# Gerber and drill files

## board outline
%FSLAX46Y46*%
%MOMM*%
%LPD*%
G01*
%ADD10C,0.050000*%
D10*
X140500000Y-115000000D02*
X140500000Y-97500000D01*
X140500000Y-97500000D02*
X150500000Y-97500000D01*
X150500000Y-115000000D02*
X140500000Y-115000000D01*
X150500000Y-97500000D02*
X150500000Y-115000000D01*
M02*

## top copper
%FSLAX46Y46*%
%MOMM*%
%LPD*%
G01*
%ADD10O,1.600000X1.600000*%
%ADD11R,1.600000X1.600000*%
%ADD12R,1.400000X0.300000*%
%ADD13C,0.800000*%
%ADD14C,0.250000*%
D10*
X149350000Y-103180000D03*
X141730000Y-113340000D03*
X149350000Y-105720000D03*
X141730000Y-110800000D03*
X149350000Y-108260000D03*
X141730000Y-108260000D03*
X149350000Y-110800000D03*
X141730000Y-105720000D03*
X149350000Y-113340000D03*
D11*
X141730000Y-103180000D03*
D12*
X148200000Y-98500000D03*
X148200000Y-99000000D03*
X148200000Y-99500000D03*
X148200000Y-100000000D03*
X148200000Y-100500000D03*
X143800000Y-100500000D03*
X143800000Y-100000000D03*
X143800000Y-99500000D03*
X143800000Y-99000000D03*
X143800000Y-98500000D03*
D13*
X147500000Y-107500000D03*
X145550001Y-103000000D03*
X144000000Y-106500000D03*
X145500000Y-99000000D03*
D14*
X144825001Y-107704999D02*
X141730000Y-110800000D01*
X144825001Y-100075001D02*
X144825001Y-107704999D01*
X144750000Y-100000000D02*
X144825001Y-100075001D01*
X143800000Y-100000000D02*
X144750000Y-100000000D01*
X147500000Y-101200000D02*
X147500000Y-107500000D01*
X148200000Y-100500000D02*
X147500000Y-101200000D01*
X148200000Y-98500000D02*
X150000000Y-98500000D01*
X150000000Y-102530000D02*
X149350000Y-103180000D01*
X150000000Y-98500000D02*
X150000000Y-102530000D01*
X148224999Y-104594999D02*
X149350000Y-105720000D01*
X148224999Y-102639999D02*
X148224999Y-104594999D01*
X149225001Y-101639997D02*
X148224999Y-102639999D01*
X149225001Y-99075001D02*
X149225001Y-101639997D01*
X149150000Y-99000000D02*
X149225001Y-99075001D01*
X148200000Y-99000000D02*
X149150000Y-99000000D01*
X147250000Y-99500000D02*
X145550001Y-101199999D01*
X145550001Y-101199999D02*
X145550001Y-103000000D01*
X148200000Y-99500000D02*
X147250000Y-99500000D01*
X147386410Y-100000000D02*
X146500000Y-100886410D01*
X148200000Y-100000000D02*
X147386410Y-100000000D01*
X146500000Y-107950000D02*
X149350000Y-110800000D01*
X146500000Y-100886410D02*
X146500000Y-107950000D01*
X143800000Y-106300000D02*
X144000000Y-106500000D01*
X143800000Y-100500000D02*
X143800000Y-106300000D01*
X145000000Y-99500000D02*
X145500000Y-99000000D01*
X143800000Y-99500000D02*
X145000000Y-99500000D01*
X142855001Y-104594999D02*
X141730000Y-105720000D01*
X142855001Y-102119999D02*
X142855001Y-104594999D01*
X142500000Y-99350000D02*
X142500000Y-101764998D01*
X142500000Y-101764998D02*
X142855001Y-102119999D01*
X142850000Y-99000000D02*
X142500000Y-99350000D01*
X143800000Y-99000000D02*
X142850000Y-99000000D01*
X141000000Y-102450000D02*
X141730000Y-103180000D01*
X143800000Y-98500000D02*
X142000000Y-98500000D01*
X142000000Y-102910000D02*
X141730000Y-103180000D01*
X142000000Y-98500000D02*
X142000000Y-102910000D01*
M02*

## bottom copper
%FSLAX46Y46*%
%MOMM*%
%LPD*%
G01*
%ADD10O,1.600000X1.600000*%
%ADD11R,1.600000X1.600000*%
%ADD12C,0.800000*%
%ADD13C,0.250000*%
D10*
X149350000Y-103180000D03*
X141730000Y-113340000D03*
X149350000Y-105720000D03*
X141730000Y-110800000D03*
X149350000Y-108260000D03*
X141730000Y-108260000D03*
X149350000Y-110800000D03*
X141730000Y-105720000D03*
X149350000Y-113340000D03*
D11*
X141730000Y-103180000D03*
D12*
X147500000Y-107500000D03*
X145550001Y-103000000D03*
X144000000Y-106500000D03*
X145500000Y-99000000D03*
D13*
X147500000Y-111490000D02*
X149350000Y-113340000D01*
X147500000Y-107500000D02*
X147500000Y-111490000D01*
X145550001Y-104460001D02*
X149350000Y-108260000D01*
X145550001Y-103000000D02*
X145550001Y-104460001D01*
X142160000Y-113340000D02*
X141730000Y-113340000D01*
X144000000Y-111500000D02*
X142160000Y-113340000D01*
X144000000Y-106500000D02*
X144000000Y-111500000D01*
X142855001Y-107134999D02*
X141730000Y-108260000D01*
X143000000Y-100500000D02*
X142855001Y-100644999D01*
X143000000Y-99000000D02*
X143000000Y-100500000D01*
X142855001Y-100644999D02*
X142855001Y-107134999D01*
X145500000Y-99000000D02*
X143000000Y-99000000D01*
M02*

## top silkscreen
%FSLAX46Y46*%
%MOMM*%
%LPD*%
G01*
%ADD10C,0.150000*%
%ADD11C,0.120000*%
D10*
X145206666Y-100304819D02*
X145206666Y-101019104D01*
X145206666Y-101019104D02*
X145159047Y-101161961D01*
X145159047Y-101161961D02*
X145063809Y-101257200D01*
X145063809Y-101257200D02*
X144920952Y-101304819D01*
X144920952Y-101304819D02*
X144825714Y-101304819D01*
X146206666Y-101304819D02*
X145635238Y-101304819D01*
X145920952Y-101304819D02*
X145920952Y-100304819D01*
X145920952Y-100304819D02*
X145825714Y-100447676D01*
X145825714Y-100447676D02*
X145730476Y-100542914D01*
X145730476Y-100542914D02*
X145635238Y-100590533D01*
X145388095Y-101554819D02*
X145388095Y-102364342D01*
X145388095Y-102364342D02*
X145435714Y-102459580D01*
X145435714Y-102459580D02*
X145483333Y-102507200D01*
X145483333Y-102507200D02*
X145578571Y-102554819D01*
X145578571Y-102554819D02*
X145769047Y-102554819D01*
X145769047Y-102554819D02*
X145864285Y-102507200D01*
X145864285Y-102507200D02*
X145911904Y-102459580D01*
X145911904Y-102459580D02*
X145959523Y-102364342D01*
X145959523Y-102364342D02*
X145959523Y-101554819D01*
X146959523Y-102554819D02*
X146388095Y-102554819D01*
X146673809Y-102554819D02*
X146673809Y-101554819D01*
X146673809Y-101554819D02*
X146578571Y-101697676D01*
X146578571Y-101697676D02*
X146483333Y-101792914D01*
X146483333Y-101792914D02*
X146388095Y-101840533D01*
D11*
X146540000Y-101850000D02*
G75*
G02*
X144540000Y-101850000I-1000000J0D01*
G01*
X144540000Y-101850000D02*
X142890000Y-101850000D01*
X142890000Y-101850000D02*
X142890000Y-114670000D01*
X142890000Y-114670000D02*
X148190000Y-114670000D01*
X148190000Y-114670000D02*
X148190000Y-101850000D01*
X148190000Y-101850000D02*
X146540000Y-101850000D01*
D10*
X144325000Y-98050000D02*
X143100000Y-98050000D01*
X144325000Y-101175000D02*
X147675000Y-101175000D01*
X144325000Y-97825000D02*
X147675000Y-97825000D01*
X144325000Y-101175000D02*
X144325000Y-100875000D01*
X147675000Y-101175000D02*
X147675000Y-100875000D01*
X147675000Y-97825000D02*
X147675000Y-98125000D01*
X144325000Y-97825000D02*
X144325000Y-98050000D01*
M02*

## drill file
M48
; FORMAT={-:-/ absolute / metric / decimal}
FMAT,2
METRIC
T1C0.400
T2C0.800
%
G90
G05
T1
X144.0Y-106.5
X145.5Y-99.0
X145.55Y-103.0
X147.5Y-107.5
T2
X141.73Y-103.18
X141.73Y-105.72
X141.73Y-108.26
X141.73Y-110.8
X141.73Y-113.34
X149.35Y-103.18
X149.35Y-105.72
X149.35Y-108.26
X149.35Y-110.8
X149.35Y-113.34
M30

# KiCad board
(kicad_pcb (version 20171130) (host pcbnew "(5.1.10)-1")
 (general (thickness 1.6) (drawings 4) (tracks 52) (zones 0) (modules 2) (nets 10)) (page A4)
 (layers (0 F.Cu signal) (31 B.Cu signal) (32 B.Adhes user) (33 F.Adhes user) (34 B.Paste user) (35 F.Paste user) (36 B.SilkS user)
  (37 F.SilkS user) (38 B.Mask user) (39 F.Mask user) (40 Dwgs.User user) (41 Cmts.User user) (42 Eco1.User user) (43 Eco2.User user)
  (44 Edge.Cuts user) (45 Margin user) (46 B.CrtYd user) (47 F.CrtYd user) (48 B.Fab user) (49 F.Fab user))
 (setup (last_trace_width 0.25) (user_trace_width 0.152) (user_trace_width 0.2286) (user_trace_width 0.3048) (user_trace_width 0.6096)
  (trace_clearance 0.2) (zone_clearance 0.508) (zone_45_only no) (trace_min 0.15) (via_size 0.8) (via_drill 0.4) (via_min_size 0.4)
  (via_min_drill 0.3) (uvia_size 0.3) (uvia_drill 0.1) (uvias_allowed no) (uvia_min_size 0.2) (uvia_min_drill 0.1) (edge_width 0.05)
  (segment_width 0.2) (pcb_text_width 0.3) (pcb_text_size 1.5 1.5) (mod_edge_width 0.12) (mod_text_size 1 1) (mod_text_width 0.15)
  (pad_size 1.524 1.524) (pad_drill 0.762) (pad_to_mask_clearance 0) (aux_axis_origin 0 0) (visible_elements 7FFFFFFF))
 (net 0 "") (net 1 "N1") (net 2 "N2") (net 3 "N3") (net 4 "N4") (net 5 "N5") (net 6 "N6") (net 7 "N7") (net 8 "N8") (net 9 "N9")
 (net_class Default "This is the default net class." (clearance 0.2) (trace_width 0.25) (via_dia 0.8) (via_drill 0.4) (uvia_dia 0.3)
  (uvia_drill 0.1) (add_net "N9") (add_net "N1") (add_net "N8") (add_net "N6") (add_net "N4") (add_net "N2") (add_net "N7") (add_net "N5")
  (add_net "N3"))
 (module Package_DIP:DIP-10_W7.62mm (layer F.Cu) (at 141.73 103.18)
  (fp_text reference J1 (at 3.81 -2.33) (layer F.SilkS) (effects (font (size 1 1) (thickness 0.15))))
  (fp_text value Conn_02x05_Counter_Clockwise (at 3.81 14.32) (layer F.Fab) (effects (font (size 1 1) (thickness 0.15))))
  (fp_arc (start 3.81 -1.33) (end 2.81 -1.33) (angle -180) (layer F.SilkS) (width 0.12))
  (fp_line (start 2.81 -1.33) (end 1.16 -1.33) (layer F.SilkS) (width 0.12))
  (fp_line (start 1.16 -1.33) (end 1.16 11.49) (layer F.SilkS) (width 0.12))
  (fp_line (start 1.16 11.49) (end 6.46 11.49) (layer F.SilkS) (width 0.12))
  (fp_line (start 6.46 11.49) (end 6.46 -1.33) (layer F.SilkS) (width 0.12))
  (fp_line (start 6.46 -1.33) (end 4.81 -1.33) (layer F.SilkS) (width 0.12))
  (pad 10 thru_hole oval (at 7.62 0) (size 1.6 1.6) (drill 0.8) (layers *.Cu *.Mask) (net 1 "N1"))
  (pad 5 thru_hole oval (at 0 10.16) (size 1.6 1.6) (drill 0.8) (layers *.Cu *.Mask) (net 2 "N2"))
  (pad 9 thru_hole oval (at 7.62 2.54) (size 1.6 1.6) (drill 0.8) (layers *.Cu *.Mask) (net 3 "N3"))
  (pad 4 thru_hole oval (at 0 7.62) (size 1.6 1.6) (drill 0.8) (layers *.Cu *.Mask) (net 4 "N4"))
  (pad 8 thru_hole oval (at 7.62 5.08) (size 1.6 1.6) (drill 0.8) (layers *.Cu *.Mask) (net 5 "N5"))
  (pad 3 thru_hole oval (at 0 5.08) (size 1.6 1.6) (drill 0.8) (layers *.Cu *.Mask) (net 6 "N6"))
  (pad 7 thru_hole oval (at 7.62 7.62) (size 1.6 1.6) (drill 0.8) (layers *.Cu *.Mask) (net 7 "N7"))
  (pad 2 thru_hole oval (at 0 2.54) (size 1.6 1.6) (drill 0.8) (layers *.Cu *.Mask) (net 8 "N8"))
  (pad 6 thru_hole oval (at 7.62 10.16) (size 1.6 1.6) (drill 0.8) (layers *.Cu *.Mask) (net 4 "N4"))
  (pad 1 thru_hole rect (at 0 0) (size 1.6 1.6) (drill 0.8) (layers *.Cu *.Mask) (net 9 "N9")))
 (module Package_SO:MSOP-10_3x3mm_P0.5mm (layer F.Cu) (at 146 99.5)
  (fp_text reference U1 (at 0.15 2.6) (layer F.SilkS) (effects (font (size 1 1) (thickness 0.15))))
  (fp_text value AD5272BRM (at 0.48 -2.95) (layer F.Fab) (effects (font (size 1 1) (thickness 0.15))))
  (fp_line (start -1.675 -1.45) (end -2.9 -1.45) (layer F.SilkS) (width 0.15))
  (fp_line (start -1.675 1.675) (end 1.675 1.675) (layer F.SilkS) (width 0.15))
  (fp_line (start -1.675 -1.675) (end 1.675 -1.675) (layer F.SilkS) (width 0.15))
  (fp_line (start -1.675 1.675) (end -1.675 1.375) (layer F.SilkS) (width 0.15))
  (fp_line (start 1.675 1.675) (end 1.675 1.375) (layer F.SilkS) (width 0.15))
  (fp_line (start 1.675 -1.675) (end 1.675 -1.375) (layer F.SilkS) (width 0.15))
  (fp_line (start -1.675 -1.675) (end -1.675 -1.45) (layer F.SilkS) (width 0.15))
  (pad 10 smd rect (at 2.2 -1) (size 1.4 0.3) (layers F.Cu F.Paste F.Mask) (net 1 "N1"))
  (pad 9 smd rect (at 2.2 -0.5) (size 1.4 0.3) (layers F.Cu F.Paste F.Mask) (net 3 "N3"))
  (pad 8 smd rect (at 2.2 0) (size 1.4 0.3) (layers F.Cu F.Paste F.Mask) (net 5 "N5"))
  (pad 7 smd rect (at 2.2 0.5) (size 1.4 0.3) (layers F.Cu F.Paste F.Mask) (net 7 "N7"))
  (pad 6 smd rect (at 2.2 1) (size 1.4 0.3) (layers F.Cu F.Paste F.Mask) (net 4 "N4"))
  (pad 5 smd rect (at -2.2 1) (size 1.4 0.3) (layers F.Cu F.Paste F.Mask) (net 2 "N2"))
  (pad 4 smd rect (at -2.2 0.5) (size 1.4 0.3) (layers F.Cu F.Paste F.Mask) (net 4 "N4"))
  (pad 3 smd rect (at -2.2 0) (size 1.4 0.3) (layers F.Cu F.Paste F.Mask) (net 6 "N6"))
  (pad 2 smd rect (at -2.2 -0.5) (size 1.4 0.3) (layers F.Cu F.Paste F.Mask) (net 8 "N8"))
  (pad 1 smd rect (at -2.2 -1) (size 1.4 0.3) (layers F.Cu F.Paste F.Mask) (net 9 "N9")))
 (gr_line (start 140.5 115) (end 140.5 97.5) (layer Edge.Cuts) (width 0.05))
 (gr_line (start 140.5 97.5) (end 150.5 97.5) (layer Edge.Cuts) (width 0.05))
 (gr_line (start 150.5 115) (end 140.5 115) (layer Edge.Cuts) (width 0.05))
 (gr_line (start 150.5 97.5) (end 150.5 115) (layer Edge.Cuts) (width 0.05))
 (segment (start 144.825001 107.704999) (end 141.73 110.8) (width 0.25) (layer F.Cu) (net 4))
 (segment (start 144.825001 100.075001) (end 144.825001 107.704999) (width 0.25) (layer F.Cu) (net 4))
 (segment (start 144.75 100) (end 144.825001 100.075001) (width 0.25) (layer F.Cu) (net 4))
 (segment (start 143.8 100) (end 144.75 100) (width 0.25) (layer F.Cu) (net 4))
 (segment (start 147.5 101.2) (end 147.5 107.5) (width 0.25) (layer F.Cu) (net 4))
 (via (at 147.5 107.5) (size 0.8) (drill 0.4) (layers F.Cu B.Cu) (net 4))
 (segment (start 148.2 100.5) (end 147.5 101.2) (width 0.25) (layer F.Cu) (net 4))
 (segment (start 147.5 111.49) (end 149.35 113.34) (width 0.25) (layer B.Cu) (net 4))
 (segment (start 147.5 107.5) (end 147.5 111.49) (width 0.25) (layer B.Cu) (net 4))
 (segment (start 148.2 98.5) (end 150 98.5) (width 0.25) (layer F.Cu) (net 1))
 (segment (start 150 102.53) (end 149.35 103.18) (width 0.25) (layer F.Cu) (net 1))
 (segment (start 150 98.5) (end 150 102.53) (width 0.25) (layer F.Cu) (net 1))
 (segment (start 148.224999 104.594999) (end 149.35 105.72) (width 0.25) (layer F.Cu) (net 3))
 (segment (start 148.224999 102.639999) (end 148.224999 104.594999) (width 0.25) (layer F.Cu) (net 3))
 (segment (start 149.225001 101.639997) (end 148.224999 102.639999) (width 0.25) (layer F.Cu) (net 3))
 (segment (start 149.225001 99.075001) (end 149.225001 101.639997) (width 0.25) (layer F.Cu) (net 3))
 (segment (start 149.15 99) (end 149.225001 99.075001) (width 0.25) (layer F.Cu) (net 3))
 (segment (start 148.2 99) (end 149.15 99) (width 0.25) (layer F.Cu) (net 3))
 (via (at 145.550001 103) (size 0.8) (drill 0.4) (layers F.Cu B.Cu) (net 5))
 (segment (start 147.25 99.5) (end 145.550001 101.199999) (width 0.25) (layer F.Cu) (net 5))
 (segment (start 145.550001 101.199999) (end 145.550001 103) (width 0.25) (layer F.Cu) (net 5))
 (segment (start 148.2 99.5) (end 147.25 99.5) (width 0.25) (layer F.Cu) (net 5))
 (segment (start 145.550001 104.460001) (end 149.35 108.26) (width 0.25) (layer B.Cu) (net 5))
 (segment (start 145.550001 103) (end 145.550001 104.460001) (width 0.25) (layer B.Cu) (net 5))
 (segment (start 147.38641 100) (end 146.5 100.88641) (width 0.25) (layer F.Cu) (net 7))
 (segment (start 148.2 100) (end 147.38641 100) (width 0.25) (layer F.Cu) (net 7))
 (segment (start 146.5 107.95) (end 149.35 110.8) (width 0.25) (layer F.Cu) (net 7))
 (segment (start 146.5 100.88641) (end 146.5 107.95) (width 0.25) (layer F.Cu) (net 7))
 (via (at 144 106.5) (size 0.8) (drill 0.4) (layers F.Cu B.Cu) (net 2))
 (segment (start 143.8 106.3) (end 144 106.5) (width 0.25) (layer F.Cu) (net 2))
 (segment (start 143.8 100.5) (end 143.8 106.3) (width 0.25) (layer F.Cu) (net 2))
 (segment (start 142.16 113.34) (end 141.73 113.34) (width 0.25) (layer B.Cu) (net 2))
 (segment (start 144 111.5) (end 142.16 113.34) (width 0.25) (layer B.Cu) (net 2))
 (segment (start 144 106.5) (end 144 111.5) (width 0.25) (layer B.Cu) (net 2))
 (segment (start 145 99.5) (end 145.5 99) (width 0.25) (layer F.Cu) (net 6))
 (via (at 145.5 99) (size 0.8) (drill 0.4) (layers F.Cu B.Cu) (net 6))
 (segment (start 143.8 99.5) (end 145 99.5) (width 0.25) (layer F.Cu) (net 6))
 (segment (start 142.855001 107.134999) (end 141.73 108.26) (width 0.25) (layer B.Cu) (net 6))
 (segment (start 143 100.5) (end 142.855001 100.644999) (width 0.25) (layer B.Cu) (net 6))
 (segment (start 143 99) (end 143 100.5) (width 0.25) (layer B.Cu) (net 6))
 (segment (start 142.855001 100.644999) (end 142.855001 107.134999) (width 0.25) (layer B.Cu) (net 6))
 (segment (start 145.5 99) (end 143 99) (width 0.25) (layer B.Cu) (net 6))
 (segment (start 142.855001 104.594999) (end 141.73 105.72) (width 0.25) (layer F.Cu) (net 8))
 (segment (start 142.855001 102.119999) (end 142.855001 104.594999) (width 0.25) (layer F.Cu) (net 8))
 (segment (start 142.5 99.35) (end 142.5 101.764998) (width 0.25) (layer F.Cu) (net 8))
 (segment (start 142.5 101.764998) (end 142.855001 102.119999) (width 0.25) (layer F.Cu) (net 8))
 (segment (start 142.85 99) (end 142.5 99.35) (width 0.25) (layer F.Cu) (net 8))
 (segment (start 143.8 99) (end 142.85 99) (width 0.25) (layer F.Cu) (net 8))
 (segment (start 141 102.45) (end 141.73 103.18) (width 0.25) (layer F.Cu) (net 9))
 (segment (start 143.8 98.5) (end 142 98.5) (width 0.25) (layer F.Cu) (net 9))
 (segment (start 142 102.91) (end 141.73 103.18) (width 0.25) (layer F.Cu) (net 9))
 (segment (start 142 98.5) (end 142 102.91) (width 0.25) (layer F.Cu) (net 9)))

